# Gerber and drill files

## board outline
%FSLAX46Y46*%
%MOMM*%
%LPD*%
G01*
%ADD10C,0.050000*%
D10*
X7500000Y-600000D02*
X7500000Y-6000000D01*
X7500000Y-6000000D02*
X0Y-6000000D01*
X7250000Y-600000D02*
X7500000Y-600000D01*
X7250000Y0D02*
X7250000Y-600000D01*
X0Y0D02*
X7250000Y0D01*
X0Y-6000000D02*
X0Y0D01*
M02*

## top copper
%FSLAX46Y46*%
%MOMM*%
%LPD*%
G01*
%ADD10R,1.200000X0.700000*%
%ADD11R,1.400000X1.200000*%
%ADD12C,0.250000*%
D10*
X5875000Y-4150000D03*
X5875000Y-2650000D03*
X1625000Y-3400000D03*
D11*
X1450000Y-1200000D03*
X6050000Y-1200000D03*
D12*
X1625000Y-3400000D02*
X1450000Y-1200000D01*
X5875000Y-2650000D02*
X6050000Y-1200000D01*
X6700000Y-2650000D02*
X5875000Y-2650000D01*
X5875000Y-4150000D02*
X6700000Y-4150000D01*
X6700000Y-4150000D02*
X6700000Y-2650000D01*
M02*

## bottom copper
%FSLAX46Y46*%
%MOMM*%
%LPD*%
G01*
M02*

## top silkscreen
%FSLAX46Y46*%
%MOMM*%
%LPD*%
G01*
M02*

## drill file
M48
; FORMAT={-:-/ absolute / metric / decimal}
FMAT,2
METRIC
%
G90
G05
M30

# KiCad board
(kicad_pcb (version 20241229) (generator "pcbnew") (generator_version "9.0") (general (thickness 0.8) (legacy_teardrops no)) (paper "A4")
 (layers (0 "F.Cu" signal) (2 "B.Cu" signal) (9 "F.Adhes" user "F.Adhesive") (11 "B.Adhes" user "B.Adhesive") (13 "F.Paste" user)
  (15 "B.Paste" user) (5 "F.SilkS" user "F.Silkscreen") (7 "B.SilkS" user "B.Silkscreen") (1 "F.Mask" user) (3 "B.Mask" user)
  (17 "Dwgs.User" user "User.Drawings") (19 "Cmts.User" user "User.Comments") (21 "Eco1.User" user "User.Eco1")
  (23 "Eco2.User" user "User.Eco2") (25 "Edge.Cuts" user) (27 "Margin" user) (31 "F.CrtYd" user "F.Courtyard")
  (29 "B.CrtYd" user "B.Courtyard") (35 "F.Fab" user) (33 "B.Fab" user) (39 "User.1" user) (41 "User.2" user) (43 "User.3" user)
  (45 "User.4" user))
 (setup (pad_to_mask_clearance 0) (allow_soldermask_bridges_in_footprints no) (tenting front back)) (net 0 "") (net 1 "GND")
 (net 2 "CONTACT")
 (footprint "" (layer "F.Cu") (at 3.75 3.4)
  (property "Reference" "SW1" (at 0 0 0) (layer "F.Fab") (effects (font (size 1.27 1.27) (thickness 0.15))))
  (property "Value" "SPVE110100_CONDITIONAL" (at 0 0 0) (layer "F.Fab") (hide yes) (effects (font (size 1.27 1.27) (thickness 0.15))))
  (pad "1" smd rect (at 2.125 0.75) (size 1.2 0.7) (layers "F.Cu" "F.Mask" "F.Paste") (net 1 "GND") (thermal_bridge_angle 45))
  (pad "2" smd rect (at 2.125 -0.75) (size 1.2 0.7) (layers "F.Cu" "F.Mask" "F.Paste") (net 1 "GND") (thermal_bridge_angle 45))
  (pad "3" smd rect (at -2.125 0) (size 1.2 0.7) (layers "F.Cu" "F.Mask" "F.Paste") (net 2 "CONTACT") (thermal_bridge_angle 45)))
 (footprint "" (layer "F.Cu") (at 0 0)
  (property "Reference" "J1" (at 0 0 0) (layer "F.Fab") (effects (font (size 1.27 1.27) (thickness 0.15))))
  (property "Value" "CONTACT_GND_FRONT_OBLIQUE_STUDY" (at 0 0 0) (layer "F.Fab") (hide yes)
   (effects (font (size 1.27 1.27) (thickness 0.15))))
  (pad "1" smd rect (at 1.45 1.2) (size 1.4 1.2) (layers "F.Cu" "F.Mask") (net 2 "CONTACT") (thermal_bridge_angle 45))
  (pad "2" smd rect (at 6.05 1.2) (size 1.4 1.2) (layers "F.Cu" "F.Mask") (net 1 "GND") (thermal_bridge_angle 45)))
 (gr_line (start 7.5 0.6) (end 7.5 6) (stroke (width 0.05) (type default)) (layer "Edge.Cuts"))
 (gr_line (start 7.5 6) (end 0 6) (stroke (width 0.05) (type default)) (layer "Edge.Cuts"))
 (gr_line (start 7.25 0.6) (end 7.5 0.6) (stroke (width 0.05) (type default)) (layer "Edge.Cuts"))
 (gr_line (start 7.25 0) (end 7.25 0.6) (stroke (width 0.05) (type default)) (layer "Edge.Cuts"))
 (gr_line (start 0 0) (end 7.25 0) (stroke (width 0.05) (type default)) (layer "Edge.Cuts"))
 (gr_line (start 0 6) (end 0 0) (stroke (width 0.05) (type default)) (layer "Edge.Cuts"))
 (segment (start 1.625 3.4) (end 1.45 1.2) (width 0.25) (layer "F.Cu") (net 2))
 (segment (start 5.875 2.65) (end 6.05 1.2) (width 0.25) (layer "F.Cu") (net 1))
 (segment (start 6.7 2.65) (end 5.875 2.65) (width 0.25) (layer "F.Cu") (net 1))
 (segment (start 5.875 4.15) (end 6.7 4.15) (width 0.25) (layer "F.Cu") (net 1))
 (segment (start 6.7 4.15) (end 6.7 2.65) (width 0.25) (layer "F.Cu") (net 1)))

